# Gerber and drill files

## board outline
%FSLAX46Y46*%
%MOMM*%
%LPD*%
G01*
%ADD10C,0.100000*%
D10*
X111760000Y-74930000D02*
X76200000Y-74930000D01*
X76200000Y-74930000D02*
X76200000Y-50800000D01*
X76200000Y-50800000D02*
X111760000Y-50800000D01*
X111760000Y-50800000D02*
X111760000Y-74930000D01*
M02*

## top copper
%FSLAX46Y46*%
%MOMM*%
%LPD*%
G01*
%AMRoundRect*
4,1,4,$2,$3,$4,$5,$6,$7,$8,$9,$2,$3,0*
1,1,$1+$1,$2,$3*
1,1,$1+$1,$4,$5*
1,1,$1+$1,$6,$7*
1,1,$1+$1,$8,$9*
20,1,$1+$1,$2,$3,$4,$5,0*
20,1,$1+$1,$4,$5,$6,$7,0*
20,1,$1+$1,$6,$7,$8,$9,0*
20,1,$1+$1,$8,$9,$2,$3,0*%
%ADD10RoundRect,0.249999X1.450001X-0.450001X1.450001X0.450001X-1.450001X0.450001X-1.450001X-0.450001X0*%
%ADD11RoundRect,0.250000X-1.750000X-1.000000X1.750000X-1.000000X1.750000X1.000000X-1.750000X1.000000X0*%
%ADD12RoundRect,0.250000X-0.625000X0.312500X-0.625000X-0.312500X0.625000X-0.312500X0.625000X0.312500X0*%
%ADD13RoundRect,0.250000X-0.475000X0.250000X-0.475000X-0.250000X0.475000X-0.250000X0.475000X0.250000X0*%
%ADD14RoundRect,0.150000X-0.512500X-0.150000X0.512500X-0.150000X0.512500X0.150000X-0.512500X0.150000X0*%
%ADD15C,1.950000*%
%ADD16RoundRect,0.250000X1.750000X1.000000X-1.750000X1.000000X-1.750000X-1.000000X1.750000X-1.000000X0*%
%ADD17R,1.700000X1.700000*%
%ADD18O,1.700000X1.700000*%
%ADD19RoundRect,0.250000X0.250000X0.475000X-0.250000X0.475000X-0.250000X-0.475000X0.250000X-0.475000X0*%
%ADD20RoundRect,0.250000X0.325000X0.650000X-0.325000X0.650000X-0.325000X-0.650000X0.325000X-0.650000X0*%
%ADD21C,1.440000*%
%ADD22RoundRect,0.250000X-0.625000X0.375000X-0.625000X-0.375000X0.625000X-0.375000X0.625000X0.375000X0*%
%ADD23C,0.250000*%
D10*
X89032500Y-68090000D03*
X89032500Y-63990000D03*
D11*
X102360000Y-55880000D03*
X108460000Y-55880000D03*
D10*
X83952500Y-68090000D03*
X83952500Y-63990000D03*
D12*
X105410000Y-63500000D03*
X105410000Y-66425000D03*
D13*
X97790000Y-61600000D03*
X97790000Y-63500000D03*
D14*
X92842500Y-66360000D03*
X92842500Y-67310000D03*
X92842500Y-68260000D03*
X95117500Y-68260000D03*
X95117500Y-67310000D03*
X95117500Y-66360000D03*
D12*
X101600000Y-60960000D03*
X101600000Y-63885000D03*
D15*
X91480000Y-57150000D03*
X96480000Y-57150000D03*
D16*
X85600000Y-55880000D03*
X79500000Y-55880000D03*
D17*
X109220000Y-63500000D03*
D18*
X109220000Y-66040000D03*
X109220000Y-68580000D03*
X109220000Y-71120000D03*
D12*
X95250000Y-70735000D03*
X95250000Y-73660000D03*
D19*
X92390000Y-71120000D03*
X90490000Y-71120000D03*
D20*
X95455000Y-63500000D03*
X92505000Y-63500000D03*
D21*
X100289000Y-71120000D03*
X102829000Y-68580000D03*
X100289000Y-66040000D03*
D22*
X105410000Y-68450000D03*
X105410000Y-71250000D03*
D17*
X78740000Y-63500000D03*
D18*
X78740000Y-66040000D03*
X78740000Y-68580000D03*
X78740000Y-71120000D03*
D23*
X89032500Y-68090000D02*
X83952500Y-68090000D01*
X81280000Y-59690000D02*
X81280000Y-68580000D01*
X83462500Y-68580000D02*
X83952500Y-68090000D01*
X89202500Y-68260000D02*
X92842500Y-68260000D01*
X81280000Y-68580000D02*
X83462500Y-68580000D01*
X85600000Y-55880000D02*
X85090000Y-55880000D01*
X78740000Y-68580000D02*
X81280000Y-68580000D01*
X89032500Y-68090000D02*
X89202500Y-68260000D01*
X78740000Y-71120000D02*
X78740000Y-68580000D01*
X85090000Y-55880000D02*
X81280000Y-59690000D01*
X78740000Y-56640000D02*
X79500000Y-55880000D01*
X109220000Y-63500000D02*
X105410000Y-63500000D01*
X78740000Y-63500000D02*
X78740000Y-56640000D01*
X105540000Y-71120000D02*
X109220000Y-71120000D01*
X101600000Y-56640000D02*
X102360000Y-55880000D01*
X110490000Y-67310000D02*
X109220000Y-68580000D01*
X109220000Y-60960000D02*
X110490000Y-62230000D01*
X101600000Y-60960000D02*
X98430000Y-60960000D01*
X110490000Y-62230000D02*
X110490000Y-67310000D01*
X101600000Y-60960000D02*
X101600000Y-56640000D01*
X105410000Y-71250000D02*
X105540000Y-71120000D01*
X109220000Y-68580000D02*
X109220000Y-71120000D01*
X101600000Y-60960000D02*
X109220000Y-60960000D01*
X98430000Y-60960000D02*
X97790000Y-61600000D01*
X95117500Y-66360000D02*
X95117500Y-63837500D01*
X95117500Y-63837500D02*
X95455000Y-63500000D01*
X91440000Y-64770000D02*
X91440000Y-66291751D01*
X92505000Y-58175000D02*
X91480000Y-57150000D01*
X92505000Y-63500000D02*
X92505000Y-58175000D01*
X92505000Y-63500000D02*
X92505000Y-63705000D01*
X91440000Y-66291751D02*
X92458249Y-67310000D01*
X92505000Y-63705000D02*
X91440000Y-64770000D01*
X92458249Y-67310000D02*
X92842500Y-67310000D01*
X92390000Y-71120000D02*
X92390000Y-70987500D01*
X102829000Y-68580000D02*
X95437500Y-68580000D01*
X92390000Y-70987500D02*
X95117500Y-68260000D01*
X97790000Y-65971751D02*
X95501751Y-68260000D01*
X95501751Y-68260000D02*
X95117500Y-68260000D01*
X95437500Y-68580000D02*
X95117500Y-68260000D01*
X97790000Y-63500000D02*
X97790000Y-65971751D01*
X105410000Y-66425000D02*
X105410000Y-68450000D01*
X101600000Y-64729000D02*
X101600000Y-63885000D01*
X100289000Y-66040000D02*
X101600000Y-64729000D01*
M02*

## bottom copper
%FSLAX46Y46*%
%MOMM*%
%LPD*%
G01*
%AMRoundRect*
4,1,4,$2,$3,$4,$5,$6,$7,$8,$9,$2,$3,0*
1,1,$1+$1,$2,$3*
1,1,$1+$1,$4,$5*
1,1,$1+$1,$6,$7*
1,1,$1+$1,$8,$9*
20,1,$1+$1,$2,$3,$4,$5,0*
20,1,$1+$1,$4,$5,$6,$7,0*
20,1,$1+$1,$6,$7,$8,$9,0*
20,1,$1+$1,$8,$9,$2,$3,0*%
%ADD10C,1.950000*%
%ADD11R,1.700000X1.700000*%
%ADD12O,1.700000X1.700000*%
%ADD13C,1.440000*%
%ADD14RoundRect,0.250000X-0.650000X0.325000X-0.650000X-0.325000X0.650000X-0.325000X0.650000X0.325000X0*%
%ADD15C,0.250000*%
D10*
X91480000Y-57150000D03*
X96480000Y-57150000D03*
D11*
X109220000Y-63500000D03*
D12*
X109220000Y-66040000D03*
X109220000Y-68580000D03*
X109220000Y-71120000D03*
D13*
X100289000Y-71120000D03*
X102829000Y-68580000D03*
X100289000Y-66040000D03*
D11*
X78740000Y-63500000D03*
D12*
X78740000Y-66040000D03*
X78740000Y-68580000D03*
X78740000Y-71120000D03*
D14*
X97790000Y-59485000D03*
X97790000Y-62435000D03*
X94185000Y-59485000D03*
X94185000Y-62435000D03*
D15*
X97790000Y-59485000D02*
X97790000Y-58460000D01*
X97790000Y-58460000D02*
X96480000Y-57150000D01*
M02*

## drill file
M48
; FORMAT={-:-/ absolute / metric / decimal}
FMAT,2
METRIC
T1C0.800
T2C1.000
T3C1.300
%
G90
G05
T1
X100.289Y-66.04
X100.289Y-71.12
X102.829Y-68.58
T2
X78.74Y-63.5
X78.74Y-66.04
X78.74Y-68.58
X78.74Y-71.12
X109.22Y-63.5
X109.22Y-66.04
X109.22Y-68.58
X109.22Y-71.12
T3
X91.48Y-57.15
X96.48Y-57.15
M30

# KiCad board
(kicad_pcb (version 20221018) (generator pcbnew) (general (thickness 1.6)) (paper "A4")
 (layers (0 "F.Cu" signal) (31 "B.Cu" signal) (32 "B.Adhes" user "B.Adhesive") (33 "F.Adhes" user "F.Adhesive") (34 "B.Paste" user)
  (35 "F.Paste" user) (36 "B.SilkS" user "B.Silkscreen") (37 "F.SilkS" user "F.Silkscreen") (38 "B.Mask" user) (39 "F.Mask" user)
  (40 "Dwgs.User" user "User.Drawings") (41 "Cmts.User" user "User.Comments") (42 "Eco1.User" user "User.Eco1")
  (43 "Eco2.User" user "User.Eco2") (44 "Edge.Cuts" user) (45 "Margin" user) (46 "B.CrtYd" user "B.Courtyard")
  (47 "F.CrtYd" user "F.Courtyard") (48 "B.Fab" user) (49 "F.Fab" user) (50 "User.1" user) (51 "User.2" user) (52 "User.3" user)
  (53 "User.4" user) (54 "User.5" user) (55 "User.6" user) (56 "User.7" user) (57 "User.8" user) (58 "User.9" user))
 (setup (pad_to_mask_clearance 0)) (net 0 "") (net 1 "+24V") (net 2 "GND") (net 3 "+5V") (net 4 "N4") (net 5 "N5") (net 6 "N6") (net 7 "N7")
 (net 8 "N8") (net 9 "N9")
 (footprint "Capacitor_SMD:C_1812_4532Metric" (layer "F.Cu") (at 89.0325 66.04 90)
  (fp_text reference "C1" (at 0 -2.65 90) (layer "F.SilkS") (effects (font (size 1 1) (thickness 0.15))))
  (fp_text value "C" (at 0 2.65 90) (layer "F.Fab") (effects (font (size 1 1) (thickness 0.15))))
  (pad "1" smd roundrect (at -2.05 0 90) (size 1.4 3.4) (layers "F.Cu" "F.Paste" "F.Mask") (roundrect_rratio 0.178571) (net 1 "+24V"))
  (pad "2" smd roundrect (at 2.05 0 90) (size 1.4 3.4) (layers "F.Cu" "F.Paste" "F.Mask") (roundrect_rratio 0.178571) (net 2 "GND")))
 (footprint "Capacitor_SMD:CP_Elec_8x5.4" (layer "F.Cu") (at 105.41 55.88)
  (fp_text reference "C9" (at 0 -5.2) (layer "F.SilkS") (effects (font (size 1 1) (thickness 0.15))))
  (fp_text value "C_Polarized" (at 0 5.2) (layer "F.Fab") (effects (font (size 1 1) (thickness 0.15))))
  (pad "1" smd roundrect (at -3.05 0) (size 4 2.5) (layers "F.Cu" "F.Paste" "F.Mask") (roundrect_rratio 0.1) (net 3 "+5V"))
  (pad "2" smd roundrect (at 3.05 0) (size 4 2.5) (layers "F.Cu" "F.Paste" "F.Mask") (roundrect_rratio 0.1) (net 2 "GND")))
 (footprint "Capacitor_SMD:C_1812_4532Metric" (layer "F.Cu") (at 83.9525 66.04 90)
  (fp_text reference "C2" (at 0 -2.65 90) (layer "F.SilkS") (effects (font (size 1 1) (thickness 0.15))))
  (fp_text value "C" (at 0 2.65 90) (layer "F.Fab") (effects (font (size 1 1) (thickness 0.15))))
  (pad "1" smd roundrect (at -2.05 0 90) (size 1.4 3.4) (layers "F.Cu" "F.Paste" "F.Mask") (roundrect_rratio 0.178571) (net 1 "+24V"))
  (pad "2" smd roundrect (at 2.05 0 90) (size 1.4 3.4) (layers "F.Cu" "F.Paste" "F.Mask") (roundrect_rratio 0.178571) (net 2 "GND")))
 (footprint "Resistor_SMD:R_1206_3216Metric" (layer "F.Cu") (at 105.41 64.9625 -90)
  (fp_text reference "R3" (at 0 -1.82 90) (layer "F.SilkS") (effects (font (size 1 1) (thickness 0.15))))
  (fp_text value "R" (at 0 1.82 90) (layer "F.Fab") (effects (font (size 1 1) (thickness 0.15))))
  (pad "1" smd roundrect (at -1.4625 0 270) (size 1.125 1.75) (layers "F.Cu" "F.Paste" "F.Mask") (roundrect_rratio 0.222222) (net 2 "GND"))
  (pad "2" smd roundrect (at 1.4625 0 270) (size 1.125 1.75) (layers "F.Cu" "F.Paste" "F.Mask") (roundrect_rratio 0.222222) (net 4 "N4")))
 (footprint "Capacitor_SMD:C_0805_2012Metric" (layer "F.Cu") (at 97.79 62.55 -90)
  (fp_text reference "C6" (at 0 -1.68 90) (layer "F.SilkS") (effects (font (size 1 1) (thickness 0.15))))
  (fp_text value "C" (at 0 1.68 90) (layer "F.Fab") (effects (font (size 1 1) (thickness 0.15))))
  (pad "1" smd roundrect (at -0.95 0 270) (size 1 1.45) (layers "F.Cu" "F.Paste" "F.Mask") (roundrect_rratio 0.25) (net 3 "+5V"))
  (pad "2" smd roundrect (at 0.95 0 270) (size 1 1.45) (layers "F.Cu" "F.Paste" "F.Mask") (roundrect_rratio 0.25) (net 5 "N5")))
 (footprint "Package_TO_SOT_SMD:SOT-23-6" (layer "F.Cu") (at 93.98 67.31)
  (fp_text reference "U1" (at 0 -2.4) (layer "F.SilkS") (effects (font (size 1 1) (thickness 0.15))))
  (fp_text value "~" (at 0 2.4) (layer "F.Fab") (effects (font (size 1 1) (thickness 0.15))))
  (pad "1" smd roundrect (at -1.1375 -0.95) (size 1.325 0.6) (layers "F.Cu" "F.Paste" "F.Mask") (roundrect_rratio 0.25) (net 2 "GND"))
  (pad "2" smd roundrect (at -1.1375 0) (size 1.325 0.6) (layers "F.Cu" "F.Paste" "F.Mask") (roundrect_rratio 0.25) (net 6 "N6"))
  (pad "3" smd roundrect (at -1.1375 0.95) (size 1.325 0.6) (layers "F.Cu" "F.Paste" "F.Mask") (roundrect_rratio 0.25) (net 1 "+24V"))
  (pad "4" smd roundrect (at 1.1375 0.95) (size 1.325 0.6) (layers "F.Cu" "F.Paste" "F.Mask") (roundrect_rratio 0.25) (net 5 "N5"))
  (pad "5" smd roundrect (at 1.1375 0) (size 1.325 0.6) (layers "F.Cu" "F.Paste" "F.Mask") (roundrect_rratio 0.25) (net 1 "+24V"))
  (pad "6" smd roundrect (at 1.1375 -0.95) (size 1.325 0.6) (layers "F.Cu" "F.Paste" "F.Mask") (roundrect_rratio 0.25) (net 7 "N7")))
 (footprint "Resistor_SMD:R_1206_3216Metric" (layer "F.Cu") (at 101.6 62.4225 -90)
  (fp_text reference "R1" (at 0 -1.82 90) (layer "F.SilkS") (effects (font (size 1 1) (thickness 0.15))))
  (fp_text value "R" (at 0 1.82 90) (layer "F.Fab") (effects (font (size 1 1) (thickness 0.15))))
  (pad "1" smd roundrect (at -1.4625 0 270) (size 1.125 1.75) (layers "F.Cu" "F.Paste" "F.Mask") (roundrect_rratio 0.222222) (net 3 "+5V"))
  (pad "2" smd roundrect (at 1.4625 0 270) (size 1.125 1.75) (layers "F.Cu" "F.Paste" "F.Mask") (roundrect_rratio 0.222222) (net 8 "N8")))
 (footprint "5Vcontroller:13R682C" (layer "F.Cu") (at 91.48 57.15 180)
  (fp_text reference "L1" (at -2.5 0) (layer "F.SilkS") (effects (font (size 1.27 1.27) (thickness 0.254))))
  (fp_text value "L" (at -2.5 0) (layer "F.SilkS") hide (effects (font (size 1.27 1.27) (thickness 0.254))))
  (pad "1" thru_hole circle (at 0 0 180) (size 1.95 1.95) (drill 1.3) (layers "*.Cu" "*.Mask") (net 6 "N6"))
  (pad "2" thru_hole circle (at -5 0 180) (size 1.95 1.95) (drill 1.3) (layers "*.Cu" "*.Mask") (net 3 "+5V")))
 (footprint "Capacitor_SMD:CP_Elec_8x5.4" (layer "F.Cu") (at 82.55 55.88 180)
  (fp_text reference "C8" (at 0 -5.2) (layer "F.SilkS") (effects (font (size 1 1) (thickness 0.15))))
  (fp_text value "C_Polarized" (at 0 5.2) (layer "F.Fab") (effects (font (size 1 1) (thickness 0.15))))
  (pad "1" smd roundrect (at -3.05 0 180) (size 4 2.5) (layers "F.Cu" "F.Paste" "F.Mask") (roundrect_rratio 0.1) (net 1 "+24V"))
  (pad "2" smd roundrect (at 3.05 0 180) (size 4 2.5) (layers "F.Cu" "F.Paste" "F.Mask") (roundrect_rratio 0.1) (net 2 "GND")))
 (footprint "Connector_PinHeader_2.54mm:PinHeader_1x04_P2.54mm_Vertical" (layer "F.Cu") (at 109.22 63.5)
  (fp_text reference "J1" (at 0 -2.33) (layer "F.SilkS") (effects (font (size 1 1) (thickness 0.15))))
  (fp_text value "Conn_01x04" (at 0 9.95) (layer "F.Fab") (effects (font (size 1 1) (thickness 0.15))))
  (pad "1" thru_hole rect (at 0 0) (size 1.7 1.7) (drill 1) (layers "*.Cu" "*.Mask") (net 2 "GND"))
  (pad "2" thru_hole oval (at 0 2.54) (size 1.7 1.7) (drill 1) (layers "*.Cu" "*.Mask") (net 2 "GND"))
  (pad "3" thru_hole oval (at 0 5.08) (size 1.7 1.7) (drill 1) (layers "*.Cu" "*.Mask") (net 3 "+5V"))
  (pad "4" thru_hole oval (at 0 7.62) (size 1.7 1.7) (drill 1) (layers "*.Cu" "*.Mask") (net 3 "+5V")))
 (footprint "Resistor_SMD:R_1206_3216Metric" (layer "F.Cu") (at 95.25 72.1975 -90)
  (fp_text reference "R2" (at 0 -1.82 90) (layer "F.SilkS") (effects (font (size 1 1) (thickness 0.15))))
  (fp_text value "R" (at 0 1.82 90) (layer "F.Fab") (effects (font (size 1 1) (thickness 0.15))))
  (pad "1" smd roundrect (at -1.4625 0 270) (size 1.125 1.75) (layers "F.Cu" "F.Paste" "F.Mask") (roundrect_rratio 0.222222) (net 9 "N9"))
  (pad "2" smd roundrect (at 1.4625 0 270) (size 1.125 1.75) (layers "F.Cu" "F.Paste" "F.Mask") (roundrect_rratio 0.222222) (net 2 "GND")))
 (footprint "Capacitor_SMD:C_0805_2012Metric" (layer "F.Cu") (at 91.44 71.12 180)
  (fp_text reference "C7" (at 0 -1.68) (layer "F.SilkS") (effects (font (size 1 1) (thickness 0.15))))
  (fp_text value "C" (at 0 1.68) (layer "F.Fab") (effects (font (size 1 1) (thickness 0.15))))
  (pad "1" smd roundrect (at -0.95 0 180) (size 1 1.45) (layers "F.Cu" "F.Paste" "F.Mask") (roundrect_rratio 0.25) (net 5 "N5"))
  (pad "2" smd roundrect (at 0.95 0 180) (size 1 1.45) (layers "F.Cu" "F.Paste" "F.Mask") (roundrect_rratio 0.25) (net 2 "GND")))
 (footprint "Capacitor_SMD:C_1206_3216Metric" (layer "F.Cu") (at 93.98 63.5 180)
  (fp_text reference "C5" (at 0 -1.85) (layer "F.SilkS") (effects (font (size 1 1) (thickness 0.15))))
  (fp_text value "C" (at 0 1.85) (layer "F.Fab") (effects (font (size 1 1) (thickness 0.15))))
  (pad "1" smd roundrect (at -1.475 0 180) (size 1.15 1.8) (layers "F.Cu" "F.Paste" "F.Mask") (roundrect_rratio 0.217391) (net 7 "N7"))
  (pad "2" smd roundrect (at 1.475 0 180) (size 1.15 1.8) (layers "F.Cu" "F.Paste" "F.Mask") (roundrect_rratio 0.217391) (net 6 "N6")))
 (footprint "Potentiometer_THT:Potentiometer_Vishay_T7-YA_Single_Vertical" (layer "F.Cu") (at 100.289 71.12)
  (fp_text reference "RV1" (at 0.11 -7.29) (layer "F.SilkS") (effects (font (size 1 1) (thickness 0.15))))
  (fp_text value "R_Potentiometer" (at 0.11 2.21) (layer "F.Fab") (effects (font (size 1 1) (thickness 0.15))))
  (pad "1" thru_hole circle (at 0 0) (size 1.44 1.44) (drill 0.8) (layers "*.Cu" "*.Mask") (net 9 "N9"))
  (pad "2" thru_hole circle (at 2.54 -2.54) (size 1.44 1.44) (drill 0.8) (layers "*.Cu" "*.Mask") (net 5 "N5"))
  (pad "3" thru_hole circle (at 0 -5.08) (size 1.44 1.44) (drill 0.8) (layers "*.Cu" "*.Mask") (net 8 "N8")))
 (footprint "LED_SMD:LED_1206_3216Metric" (layer "F.Cu") (at 105.41 69.85 -90)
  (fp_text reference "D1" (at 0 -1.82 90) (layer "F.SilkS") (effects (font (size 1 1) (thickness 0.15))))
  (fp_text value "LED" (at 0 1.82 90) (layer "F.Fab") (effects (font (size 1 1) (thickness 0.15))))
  (pad "1" smd roundrect (at -1.4 0 270) (size 1.25 1.75) (layers "F.Cu" "F.Paste" "F.Mask") (roundrect_rratio 0.2) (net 4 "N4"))
  (pad "2" smd roundrect (at 1.4 0 270) (size 1.25 1.75) (layers "F.Cu" "F.Paste" "F.Mask") (roundrect_rratio 0.2) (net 3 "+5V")))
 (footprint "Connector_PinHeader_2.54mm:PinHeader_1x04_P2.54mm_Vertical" (layer "F.Cu") (at 78.74 63.5)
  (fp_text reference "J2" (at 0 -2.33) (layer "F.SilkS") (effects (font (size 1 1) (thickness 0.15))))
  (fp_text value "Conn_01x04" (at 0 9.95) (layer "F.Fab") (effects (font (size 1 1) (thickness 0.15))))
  (pad "1" thru_hole rect (at 0 0) (size 1.7 1.7) (drill 1) (layers "*.Cu" "*.Mask") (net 2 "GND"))
  (pad "2" thru_hole oval (at 0 2.54) (size 1.7 1.7) (drill 1) (layers "*.Cu" "*.Mask") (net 2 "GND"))
  (pad "3" thru_hole oval (at 0 5.08) (size 1.7 1.7) (drill 1) (layers "*.Cu" "*.Mask") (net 1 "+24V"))
  (pad "4" thru_hole oval (at 0 7.62) (size 1.7 1.7) (drill 1) (layers "*.Cu" "*.Mask") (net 1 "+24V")))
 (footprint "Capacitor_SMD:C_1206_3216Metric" (layer "B.Cu") (at 97.79 60.96 -90)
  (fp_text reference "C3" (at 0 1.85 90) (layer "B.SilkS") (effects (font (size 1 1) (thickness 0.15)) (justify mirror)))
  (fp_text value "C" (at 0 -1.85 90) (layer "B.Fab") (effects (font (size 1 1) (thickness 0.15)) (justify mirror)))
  (pad "1" smd roundrect (at -1.475 0 270) (size 1.15 1.8) (layers "B.Cu" "B.Paste" "B.Mask") (roundrect_rratio 0.217391) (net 3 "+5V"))
  (pad "2" smd roundrect (at 1.475 0 270) (size 1.15 1.8) (layers "B.Cu" "B.Paste" "B.Mask") (roundrect_rratio 0.217391) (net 2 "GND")))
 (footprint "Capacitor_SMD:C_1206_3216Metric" (layer "B.Cu") (at 94.185 60.96 -90)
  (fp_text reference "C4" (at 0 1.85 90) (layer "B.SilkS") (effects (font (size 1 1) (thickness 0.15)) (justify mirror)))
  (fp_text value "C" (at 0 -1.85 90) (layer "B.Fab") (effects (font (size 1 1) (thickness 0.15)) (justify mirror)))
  (pad "1" smd roundrect (at -1.475 0 270) (size 1.15 1.8) (layers "B.Cu" "B.Paste" "B.Mask") (roundrect_rratio 0.217391) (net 3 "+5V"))
  (pad "2" smd roundrect (at 1.475 0 270) (size 1.15 1.8) (layers "B.Cu" "B.Paste" "B.Mask") (roundrect_rratio 0.217391) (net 2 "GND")))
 (gr_line (start 111.76 74.93) (end 76.2 74.93) (stroke (width 0.1) (type default)) (layer "Edge.Cuts"))
 (gr_line (start 76.2 74.93) (end 76.2 50.8) (stroke (width 0.1) (type default)) (layer "Edge.Cuts"))
 (gr_line (start 76.2 50.8) (end 111.76 50.8) (stroke (width 0.1) (type default)) (layer "Edge.Cuts"))
 (gr_line (start 111.76 50.8) (end 111.76 74.93) (stroke (width 0.1) (type default)) (layer "Edge.Cuts"))
 (segment (start 89.0325 68.09) (end 83.9525 68.09) (width 0.25) (layer "F.Cu") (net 1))
 (segment (start 81.28 59.69) (end 81.28 68.58) (width 0.25) (layer "F.Cu") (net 1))
 (segment (start 83.4625 68.58) (end 83.9525 68.09) (width 0.25) (layer "F.Cu") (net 1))
 (segment (start 89.2025 68.26) (end 92.8425 68.26) (width 0.25) (layer "F.Cu") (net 1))
 (segment (start 81.28 68.58) (end 83.4625 68.58) (width 0.25) (layer "F.Cu") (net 1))
 (segment (start 85.6 55.88) (end 85.09 55.88) (width 0.25) (layer "F.Cu") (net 1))
 (segment (start 78.74 68.58) (end 81.28 68.58) (width 0.25) (layer "F.Cu") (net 1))
 (segment (start 89.0325 68.09) (end 89.2025 68.26) (width 0.25) (layer "F.Cu") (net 1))
 (segment (start 78.74 71.12) (end 78.74 68.58) (width 0.25) (layer "F.Cu") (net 1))
 (segment (start 85.09 55.88) (end 81.28 59.69) (width 0.25) (layer "F.Cu") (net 1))
 (segment (start 78.74 56.64) (end 79.5 55.88) (width 0.25) (layer "F.Cu") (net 2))
 (segment (start 109.22 63.5) (end 105.41 63.5) (width 0.25) (layer "F.Cu") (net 2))
 (segment (start 78.74 63.5) (end 78.74 56.64) (width 0.25) (layer "F.Cu") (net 2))
 (segment (start 105.54 71.12) (end 109.22 71.12) (width 0.25) (layer "F.Cu") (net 3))
 (segment (start 101.6 56.64) (end 102.36 55.88) (width 0.25) (layer "F.Cu") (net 3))
 (segment (start 110.49 67.31) (end 109.22 68.58) (width 0.25) (layer "F.Cu") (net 3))
 (segment (start 109.22 60.96) (end 110.49 62.23) (width 0.25) (layer "F.Cu") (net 3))
 (segment (start 101.6 60.96) (end 98.43 60.96) (width 0.25) (layer "F.Cu") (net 3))
 (segment (start 110.49 62.23) (end 110.49 67.31) (width 0.25) (layer "F.Cu") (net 3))
 (segment (start 101.6 60.96) (end 101.6 56.64) (width 0.25) (layer "F.Cu") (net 3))
 (segment (start 105.41 71.25) (end 105.54 71.12) (width 0.25) (layer "F.Cu") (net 3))
 (segment (start 109.22 68.58) (end 109.22 71.12) (width 0.25) (layer "F.Cu") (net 3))
 (segment (start 101.6 60.96) (end 109.22 60.96) (width 0.25) (layer "F.Cu") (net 3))
 (segment (start 98.43 60.96) (end 97.79 61.6) (width 0.25) (layer "F.Cu") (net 3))
 (segment (start 97.79 59.485) (end 97.79 58.46) (width 0.25) (layer "B.Cu") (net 3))
 (segment (start 97.79 58.46) (end 96.48 57.15) (width 0.25) (layer "B.Cu") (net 3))
 (segment (start 95.1175 66.36) (end 95.1175 63.8375) (width 0.25) (layer "F.Cu") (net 7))
 (segment (start 95.1175 63.8375) (end 95.455 63.5) (width 0.25) (layer "F.Cu") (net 7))
 (segment (start 91.44 64.77) (end 91.44 66.291751) (width 0.25) (layer "F.Cu") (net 6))
 (segment (start 92.505 58.175) (end 91.48 57.15) (width 0.25) (layer "F.Cu") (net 6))
 (segment (start 92.505 63.5) (end 92.505 58.175) (width 0.25) (layer "F.Cu") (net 6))
 (segment (start 92.505 63.5) (end 92.505 63.705) (width 0.25) (layer "F.Cu") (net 6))
 (segment (start 91.44 66.291751) (end 92.458249 67.31) (width 0.25) (layer "F.Cu") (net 6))
 (segment (start 92.505 63.705) (end 91.44 64.77) (width 0.25) (layer "F.Cu") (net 6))
 (segment (start 92.458249 67.31) (end 92.8425 67.31) (width 0.25) (layer "F.Cu") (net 6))
 (segment (start 92.39 71.12) (end 92.39 70.9875) (width 0.25) (layer "F.Cu") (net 5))
 (segment (start 102.829 68.58) (end 95.4375 68.58) (width 0.25) (layer "F.Cu") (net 5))
 (segment (start 92.39 70.9875) (end 95.1175 68.26) (width 0.25) (layer "F.Cu") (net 5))
 (segment (start 97.79 65.971751) (end 95.501751 68.26) (width 0.25) (layer "F.Cu") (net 5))
 (segment (start 95.501751 68.26) (end 95.1175 68.26) (width 0.25) (layer "F.Cu") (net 5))
 (segment (start 95.4375 68.58) (end 95.1175 68.26) (width 0.25) (layer "F.Cu") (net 5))
 (segment (start 97.79 63.5) (end 97.79 65.971751) (width 0.25) (layer "F.Cu") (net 5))
 (segment (start 105.41 66.425) (end 105.41 68.45) (width 0.25) (layer "F.Cu") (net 4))
 (segment (start 101.6 64.729) (end 101.6 63.885) (width 0.25) (layer "F.Cu") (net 8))
 (segment (start 100.289 66.04) (end 101.6 64.729) (width 0.25) (layer "F.Cu") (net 8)))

